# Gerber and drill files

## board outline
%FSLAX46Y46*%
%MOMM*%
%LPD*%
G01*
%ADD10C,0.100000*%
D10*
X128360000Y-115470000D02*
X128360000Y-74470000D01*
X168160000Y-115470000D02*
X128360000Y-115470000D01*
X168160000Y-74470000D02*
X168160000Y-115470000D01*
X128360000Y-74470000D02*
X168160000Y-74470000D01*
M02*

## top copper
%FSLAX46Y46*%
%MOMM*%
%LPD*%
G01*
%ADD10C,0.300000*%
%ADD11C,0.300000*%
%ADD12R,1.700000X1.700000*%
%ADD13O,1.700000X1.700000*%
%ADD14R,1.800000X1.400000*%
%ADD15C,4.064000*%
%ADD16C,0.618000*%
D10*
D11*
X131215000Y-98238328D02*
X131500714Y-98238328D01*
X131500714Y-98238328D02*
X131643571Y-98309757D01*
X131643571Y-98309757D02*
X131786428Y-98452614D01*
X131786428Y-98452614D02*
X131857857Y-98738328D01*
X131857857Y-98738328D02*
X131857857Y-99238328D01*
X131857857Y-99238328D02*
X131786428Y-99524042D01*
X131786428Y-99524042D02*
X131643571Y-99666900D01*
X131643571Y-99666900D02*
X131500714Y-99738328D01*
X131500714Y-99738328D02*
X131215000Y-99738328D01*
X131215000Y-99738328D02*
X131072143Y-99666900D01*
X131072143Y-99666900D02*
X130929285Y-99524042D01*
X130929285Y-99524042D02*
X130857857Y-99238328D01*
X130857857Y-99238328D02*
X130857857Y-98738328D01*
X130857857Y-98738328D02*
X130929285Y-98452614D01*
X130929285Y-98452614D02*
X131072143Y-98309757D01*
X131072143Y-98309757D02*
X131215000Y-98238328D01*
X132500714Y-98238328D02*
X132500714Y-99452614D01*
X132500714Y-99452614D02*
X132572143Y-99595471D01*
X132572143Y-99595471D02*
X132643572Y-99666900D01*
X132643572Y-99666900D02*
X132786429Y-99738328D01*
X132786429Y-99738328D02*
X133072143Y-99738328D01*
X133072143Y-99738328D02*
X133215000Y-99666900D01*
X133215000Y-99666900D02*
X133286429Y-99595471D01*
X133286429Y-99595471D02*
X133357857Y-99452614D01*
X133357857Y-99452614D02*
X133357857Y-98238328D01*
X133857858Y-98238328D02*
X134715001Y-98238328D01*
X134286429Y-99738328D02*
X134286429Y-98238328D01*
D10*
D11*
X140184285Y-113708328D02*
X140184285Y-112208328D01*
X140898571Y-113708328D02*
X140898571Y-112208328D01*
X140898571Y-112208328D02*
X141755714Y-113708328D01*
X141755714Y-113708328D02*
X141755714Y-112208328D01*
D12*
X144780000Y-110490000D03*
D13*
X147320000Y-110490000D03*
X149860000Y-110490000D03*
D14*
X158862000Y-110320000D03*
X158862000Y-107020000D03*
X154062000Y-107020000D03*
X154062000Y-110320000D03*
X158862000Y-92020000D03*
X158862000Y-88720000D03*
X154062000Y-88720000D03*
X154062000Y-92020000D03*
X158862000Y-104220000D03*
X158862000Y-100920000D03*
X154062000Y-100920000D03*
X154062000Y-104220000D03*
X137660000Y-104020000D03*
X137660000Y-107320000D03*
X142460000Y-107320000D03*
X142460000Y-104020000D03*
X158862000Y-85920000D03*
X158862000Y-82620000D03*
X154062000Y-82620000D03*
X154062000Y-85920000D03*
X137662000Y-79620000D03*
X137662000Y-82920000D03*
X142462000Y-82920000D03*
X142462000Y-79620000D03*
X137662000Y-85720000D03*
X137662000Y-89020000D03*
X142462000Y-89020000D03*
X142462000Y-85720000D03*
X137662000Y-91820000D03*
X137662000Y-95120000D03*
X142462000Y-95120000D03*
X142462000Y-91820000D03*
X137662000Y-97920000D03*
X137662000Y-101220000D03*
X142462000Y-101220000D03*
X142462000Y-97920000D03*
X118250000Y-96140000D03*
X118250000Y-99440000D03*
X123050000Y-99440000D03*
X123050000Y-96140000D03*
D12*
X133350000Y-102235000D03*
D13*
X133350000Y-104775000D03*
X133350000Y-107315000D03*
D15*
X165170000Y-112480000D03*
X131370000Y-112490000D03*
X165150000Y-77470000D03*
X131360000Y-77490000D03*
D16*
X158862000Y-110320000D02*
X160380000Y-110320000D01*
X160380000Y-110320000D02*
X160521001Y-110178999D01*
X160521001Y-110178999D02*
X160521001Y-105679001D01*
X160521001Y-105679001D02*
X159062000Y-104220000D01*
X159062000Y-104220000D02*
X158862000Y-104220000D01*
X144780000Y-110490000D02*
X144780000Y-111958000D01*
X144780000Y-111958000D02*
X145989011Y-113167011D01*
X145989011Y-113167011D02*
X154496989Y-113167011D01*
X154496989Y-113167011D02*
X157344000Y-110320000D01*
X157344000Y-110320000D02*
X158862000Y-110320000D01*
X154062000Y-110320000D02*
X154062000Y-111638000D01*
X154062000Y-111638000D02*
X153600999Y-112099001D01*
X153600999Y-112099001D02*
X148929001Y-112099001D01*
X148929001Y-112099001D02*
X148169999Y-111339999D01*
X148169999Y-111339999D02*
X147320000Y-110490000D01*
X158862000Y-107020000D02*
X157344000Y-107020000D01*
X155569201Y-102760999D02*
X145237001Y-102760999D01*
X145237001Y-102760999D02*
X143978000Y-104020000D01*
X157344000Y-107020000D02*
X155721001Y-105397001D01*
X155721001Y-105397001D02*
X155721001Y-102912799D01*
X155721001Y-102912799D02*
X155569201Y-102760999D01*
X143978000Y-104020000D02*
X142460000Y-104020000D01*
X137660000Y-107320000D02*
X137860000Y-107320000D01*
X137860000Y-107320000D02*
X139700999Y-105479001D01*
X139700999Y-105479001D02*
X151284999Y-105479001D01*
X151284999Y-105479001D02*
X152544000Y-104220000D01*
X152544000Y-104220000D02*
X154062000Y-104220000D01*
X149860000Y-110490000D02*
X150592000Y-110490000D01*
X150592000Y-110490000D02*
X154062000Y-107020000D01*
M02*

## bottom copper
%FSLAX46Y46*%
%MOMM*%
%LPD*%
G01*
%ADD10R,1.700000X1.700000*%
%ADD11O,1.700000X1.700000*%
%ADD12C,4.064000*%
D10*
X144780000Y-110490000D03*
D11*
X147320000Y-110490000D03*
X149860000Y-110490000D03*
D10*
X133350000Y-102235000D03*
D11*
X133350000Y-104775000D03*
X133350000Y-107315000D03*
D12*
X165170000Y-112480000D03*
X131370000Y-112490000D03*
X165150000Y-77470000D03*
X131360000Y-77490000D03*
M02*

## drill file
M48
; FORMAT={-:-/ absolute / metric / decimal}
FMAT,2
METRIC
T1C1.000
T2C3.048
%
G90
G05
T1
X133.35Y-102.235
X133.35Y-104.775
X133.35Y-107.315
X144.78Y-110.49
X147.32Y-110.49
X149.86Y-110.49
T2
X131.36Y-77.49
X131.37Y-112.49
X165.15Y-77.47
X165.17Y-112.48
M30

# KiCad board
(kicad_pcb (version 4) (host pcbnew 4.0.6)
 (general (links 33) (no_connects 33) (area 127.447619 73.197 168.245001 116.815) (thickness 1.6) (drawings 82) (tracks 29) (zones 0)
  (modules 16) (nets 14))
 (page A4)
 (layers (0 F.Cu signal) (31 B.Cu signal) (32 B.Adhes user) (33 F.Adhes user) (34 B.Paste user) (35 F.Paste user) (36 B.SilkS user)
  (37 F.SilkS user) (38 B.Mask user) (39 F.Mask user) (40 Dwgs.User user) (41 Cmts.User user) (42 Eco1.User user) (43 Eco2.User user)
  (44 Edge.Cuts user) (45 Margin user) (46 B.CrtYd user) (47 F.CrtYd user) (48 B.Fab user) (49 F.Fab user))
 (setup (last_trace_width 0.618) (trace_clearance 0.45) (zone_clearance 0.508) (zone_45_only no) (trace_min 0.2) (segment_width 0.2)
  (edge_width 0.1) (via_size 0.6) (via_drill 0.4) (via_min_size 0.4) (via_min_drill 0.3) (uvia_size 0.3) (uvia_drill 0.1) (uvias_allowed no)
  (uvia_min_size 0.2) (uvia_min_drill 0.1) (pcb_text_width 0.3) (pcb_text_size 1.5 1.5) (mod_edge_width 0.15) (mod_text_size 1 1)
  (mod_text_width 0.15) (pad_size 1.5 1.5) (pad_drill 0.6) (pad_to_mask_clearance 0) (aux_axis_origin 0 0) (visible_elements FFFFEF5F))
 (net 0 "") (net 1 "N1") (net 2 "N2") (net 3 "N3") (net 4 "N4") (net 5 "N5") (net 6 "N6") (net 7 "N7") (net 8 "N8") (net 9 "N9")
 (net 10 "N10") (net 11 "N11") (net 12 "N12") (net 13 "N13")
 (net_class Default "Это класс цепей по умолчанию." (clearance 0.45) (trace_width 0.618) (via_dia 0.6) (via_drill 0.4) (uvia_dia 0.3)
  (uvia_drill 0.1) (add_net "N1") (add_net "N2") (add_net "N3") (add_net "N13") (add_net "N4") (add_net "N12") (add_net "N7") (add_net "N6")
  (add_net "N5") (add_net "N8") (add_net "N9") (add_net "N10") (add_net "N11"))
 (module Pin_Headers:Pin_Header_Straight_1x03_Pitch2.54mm (layer F.Cu) (at 144.78 110.49 90)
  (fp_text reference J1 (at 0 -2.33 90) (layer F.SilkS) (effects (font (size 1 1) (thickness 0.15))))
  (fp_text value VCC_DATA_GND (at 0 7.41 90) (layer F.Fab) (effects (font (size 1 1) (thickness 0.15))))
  (pad 1 thru_hole rect (at 0 0 90) (size 1.7 1.7) (drill 1) (layers *.Cu *.Mask) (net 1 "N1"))
  (pad 2 thru_hole oval (at 0 2.54 90) (size 1.7 1.7) (drill 1) (layers *.Cu *.Mask) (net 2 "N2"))
  (pad 3 thru_hole oval (at 0 5.08 90) (size 1.7 1.7) (drill 1) (layers *.Cu *.Mask) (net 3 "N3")))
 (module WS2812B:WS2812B (layer F.Cu) (at 156.462 108.67 270)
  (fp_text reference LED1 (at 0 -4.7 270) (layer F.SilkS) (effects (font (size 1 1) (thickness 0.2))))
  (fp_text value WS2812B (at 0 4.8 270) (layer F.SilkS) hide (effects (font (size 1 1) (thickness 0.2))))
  (pad 1 smd rect (at 1.65 -2.4 270) (size 1.4 1.8) (layers F.Cu F.Paste F.Mask) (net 1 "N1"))
  (pad 2 smd rect (at -1.65 -2.4 270) (size 1.4 1.8) (layers F.Cu F.Paste F.Mask) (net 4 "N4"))
  (pad 3 smd rect (at -1.65 2.4 270) (size 1.4 1.8) (layers F.Cu F.Paste F.Mask) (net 3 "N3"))
  (pad 4 smd rect (at 1.65 2.4 270) (size 1.4 1.8) (layers F.Cu F.Paste F.Mask) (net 2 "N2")))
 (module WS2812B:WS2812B (layer F.Cu) (at 156.462 90.37 270)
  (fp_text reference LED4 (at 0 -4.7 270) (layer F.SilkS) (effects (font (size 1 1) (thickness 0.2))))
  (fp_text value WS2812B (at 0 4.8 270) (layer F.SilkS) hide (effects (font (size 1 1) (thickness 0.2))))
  (pad 1 smd rect (at 1.65 -2.4 270) (size 1.4 1.8) (layers F.Cu F.Paste F.Mask) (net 1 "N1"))
  (pad 2 smd rect (at -1.65 -2.4 270) (size 1.4 1.8) (layers F.Cu F.Paste F.Mask) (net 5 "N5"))
  (pad 3 smd rect (at -1.65 2.4 270) (size 1.4 1.8) (layers F.Cu F.Paste F.Mask) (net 3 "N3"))
  (pad 4 smd rect (at 1.65 2.4 270) (size 1.4 1.8) (layers F.Cu F.Paste F.Mask) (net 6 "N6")))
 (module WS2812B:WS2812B (layer F.Cu) (at 156.462 102.57 270)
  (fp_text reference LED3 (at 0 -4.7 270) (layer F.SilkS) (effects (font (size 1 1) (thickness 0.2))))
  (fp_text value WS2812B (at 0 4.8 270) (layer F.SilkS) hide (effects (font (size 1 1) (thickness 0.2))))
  (pad 1 smd rect (at 1.65 -2.4 270) (size 1.4 1.8) (layers F.Cu F.Paste F.Mask) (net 1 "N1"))
  (pad 2 smd rect (at -1.65 -2.4 270) (size 1.4 1.8) (layers F.Cu F.Paste F.Mask) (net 6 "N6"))
  (pad 3 smd rect (at -1.65 2.4 270) (size 1.4 1.8) (layers F.Cu F.Paste F.Mask) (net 3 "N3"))
  (pad 4 smd rect (at 1.65 2.4 270) (size 1.4 1.8) (layers F.Cu F.Paste F.Mask) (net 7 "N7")))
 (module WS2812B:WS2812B (layer F.Cu) (at 140.06 105.67 90)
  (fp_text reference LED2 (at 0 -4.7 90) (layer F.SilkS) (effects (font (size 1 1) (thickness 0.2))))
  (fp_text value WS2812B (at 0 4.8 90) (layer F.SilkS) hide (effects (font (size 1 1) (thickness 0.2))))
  (pad 1 smd rect (at 1.65 -2.4 90) (size 1.4 1.8) (layers F.Cu F.Paste F.Mask) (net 1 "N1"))
  (pad 2 smd rect (at -1.65 -2.4 90) (size 1.4 1.8) (layers F.Cu F.Paste F.Mask) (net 7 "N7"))
  (pad 3 smd rect (at -1.65 2.4 90) (size 1.4 1.8) (layers F.Cu F.Paste F.Mask) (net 3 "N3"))
  (pad 4 smd rect (at 1.65 2.4 90) (size 1.4 1.8) (layers F.Cu F.Paste F.Mask) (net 4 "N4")))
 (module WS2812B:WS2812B (layer F.Cu) (at 156.462 84.27 270)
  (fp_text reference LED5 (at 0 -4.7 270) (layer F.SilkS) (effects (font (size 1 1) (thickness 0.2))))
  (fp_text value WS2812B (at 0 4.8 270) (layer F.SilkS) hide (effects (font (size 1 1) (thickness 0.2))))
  (pad 1 smd rect (at 1.65 -2.4 270) (size 1.4 1.8) (layers F.Cu F.Paste F.Mask) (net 1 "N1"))
  (pad 2 smd rect (at -1.65 -2.4 270) (size 1.4 1.8) (layers F.Cu F.Paste F.Mask) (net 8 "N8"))
  (pad 3 smd rect (at -1.65 2.4 270) (size 1.4 1.8) (layers F.Cu F.Paste F.Mask) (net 3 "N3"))
  (pad 4 smd rect (at 1.65 2.4 270) (size 1.4 1.8) (layers F.Cu F.Paste F.Mask) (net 5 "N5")))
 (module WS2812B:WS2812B (layer F.Cu) (at 140.062 81.27 90)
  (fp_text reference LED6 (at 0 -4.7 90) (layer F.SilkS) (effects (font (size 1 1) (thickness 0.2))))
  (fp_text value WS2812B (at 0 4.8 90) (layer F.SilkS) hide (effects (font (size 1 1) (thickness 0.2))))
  (pad 1 smd rect (at 1.65 -2.4 90) (size 1.4 1.8) (layers F.Cu F.Paste F.Mask) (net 1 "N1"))
  (pad 2 smd rect (at -1.65 -2.4 90) (size 1.4 1.8) (layers F.Cu F.Paste F.Mask) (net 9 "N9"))
  (pad 3 smd rect (at -1.65 2.4 90) (size 1.4 1.8) (layers F.Cu F.Paste F.Mask) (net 3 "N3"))
  (pad 4 smd rect (at 1.65 2.4 90) (size 1.4 1.8) (layers F.Cu F.Paste F.Mask) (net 8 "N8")))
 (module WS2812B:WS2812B (layer F.Cu) (at 140.062 87.37 90)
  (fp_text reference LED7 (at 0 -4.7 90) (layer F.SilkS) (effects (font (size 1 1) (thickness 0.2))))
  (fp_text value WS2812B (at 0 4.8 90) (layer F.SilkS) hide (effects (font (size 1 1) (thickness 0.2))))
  (pad 1 smd rect (at 1.65 -2.4 90) (size 1.4 1.8) (layers F.Cu F.Paste F.Mask) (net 1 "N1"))
  (pad 2 smd rect (at -1.65 -2.4 90) (size 1.4 1.8) (layers F.Cu F.Paste F.Mask) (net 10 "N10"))
  (pad 3 smd rect (at -1.65 2.4 90) (size 1.4 1.8) (layers F.Cu F.Paste F.Mask) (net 3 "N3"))
  (pad 4 smd rect (at 1.65 2.4 90) (size 1.4 1.8) (layers F.Cu F.Paste F.Mask) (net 9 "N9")))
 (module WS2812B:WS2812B (layer F.Cu) (at 140.062 93.47 90)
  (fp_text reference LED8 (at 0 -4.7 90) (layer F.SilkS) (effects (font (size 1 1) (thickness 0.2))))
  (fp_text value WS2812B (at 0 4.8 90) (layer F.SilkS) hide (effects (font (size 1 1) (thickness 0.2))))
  (pad 1 smd rect (at 1.65 -2.4 90) (size 1.4 1.8) (layers F.Cu F.Paste F.Mask) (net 1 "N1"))
  (pad 2 smd rect (at -1.65 -2.4 90) (size 1.4 1.8) (layers F.Cu F.Paste F.Mask) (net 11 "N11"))
  (pad 3 smd rect (at -1.65 2.4 90) (size 1.4 1.8) (layers F.Cu F.Paste F.Mask) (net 3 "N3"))
  (pad 4 smd rect (at 1.65 2.4 90) (size 1.4 1.8) (layers F.Cu F.Paste F.Mask) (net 10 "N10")))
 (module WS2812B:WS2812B (layer F.Cu) (at 140.062 99.57 90)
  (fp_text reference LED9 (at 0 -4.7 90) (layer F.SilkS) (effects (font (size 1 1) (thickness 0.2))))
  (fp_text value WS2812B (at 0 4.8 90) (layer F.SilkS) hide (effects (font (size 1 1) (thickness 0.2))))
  (pad 1 smd rect (at 1.65 -2.4 90) (size 1.4 1.8) (layers F.Cu F.Paste F.Mask) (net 1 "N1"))
  (pad 2 smd rect (at -1.65 -2.4 90) (size 1.4 1.8) (layers F.Cu F.Paste F.Mask) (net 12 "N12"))
  (pad 3 smd rect (at -1.65 2.4 90) (size 1.4 1.8) (layers F.Cu F.Paste F.Mask) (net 3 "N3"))
  (pad 4 smd rect (at 1.65 2.4 90) (size 1.4 1.8) (layers F.Cu F.Paste F.Mask) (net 11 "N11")))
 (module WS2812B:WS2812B (layer F.Cu) (at 120.65 97.79 90)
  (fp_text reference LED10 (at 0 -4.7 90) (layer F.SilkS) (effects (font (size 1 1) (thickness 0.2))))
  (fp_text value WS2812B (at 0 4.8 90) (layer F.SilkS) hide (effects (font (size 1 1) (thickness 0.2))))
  (pad 1 smd rect (at 1.65 -2.4 90) (size 1.4 1.8) (layers F.Cu F.Paste F.Mask) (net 1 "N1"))
  (pad 2 smd rect (at -1.65 -2.4 90) (size 1.4 1.8) (layers F.Cu F.Paste F.Mask) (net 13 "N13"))
  (pad 3 smd rect (at -1.65 2.4 90) (size 1.4 1.8) (layers F.Cu F.Paste F.Mask) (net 3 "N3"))
  (pad 4 smd rect (at 1.65 2.4 90) (size 1.4 1.8) (layers F.Cu F.Paste F.Mask) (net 12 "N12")))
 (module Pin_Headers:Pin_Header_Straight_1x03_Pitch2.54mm (layer F.Cu) (at 133.35 102.235)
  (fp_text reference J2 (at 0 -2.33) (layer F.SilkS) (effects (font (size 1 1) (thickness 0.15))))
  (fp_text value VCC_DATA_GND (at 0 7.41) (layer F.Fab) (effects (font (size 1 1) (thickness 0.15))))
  (pad 1 thru_hole rect (at 0 0) (size 1.7 1.7) (drill 1) (layers *.Cu *.Mask) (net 1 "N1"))
  (pad 2 thru_hole oval (at 0 2.54) (size 1.7 1.7) (drill 1) (layers *.Cu *.Mask) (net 13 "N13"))
  (pad 3 thru_hole oval (at 0 5.08) (size 1.7 1.7) (drill 1) (layers *.Cu *.Mask) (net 3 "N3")))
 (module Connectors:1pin (layer F.Cu) (at 165.17 112.48)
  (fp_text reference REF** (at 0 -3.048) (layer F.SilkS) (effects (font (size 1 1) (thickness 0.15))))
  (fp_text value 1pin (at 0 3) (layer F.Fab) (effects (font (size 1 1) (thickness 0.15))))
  (pad 1 thru_hole circle (at 0 0) (size 4.064 4.064) (drill 3.048) (layers *.Cu *.Mask)))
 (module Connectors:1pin (layer F.Cu) (at 131.37 112.49)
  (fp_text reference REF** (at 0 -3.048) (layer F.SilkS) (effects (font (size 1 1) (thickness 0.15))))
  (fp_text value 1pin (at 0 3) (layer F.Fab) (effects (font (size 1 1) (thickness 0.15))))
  (pad 1 thru_hole circle (at 0 0) (size 4.064 4.064) (drill 3.048) (layers *.Cu *.Mask)))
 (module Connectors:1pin (layer F.Cu) (at 165.15 77.47)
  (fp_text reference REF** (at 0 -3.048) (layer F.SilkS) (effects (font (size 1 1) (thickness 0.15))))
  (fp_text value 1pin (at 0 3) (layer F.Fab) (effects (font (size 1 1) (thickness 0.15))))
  (pad 1 thru_hole circle (at 0 0) (size 4.064 4.064) (drill 3.048) (layers *.Cu *.Mask)))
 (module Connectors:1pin (layer F.Cu) (at 131.36 77.49)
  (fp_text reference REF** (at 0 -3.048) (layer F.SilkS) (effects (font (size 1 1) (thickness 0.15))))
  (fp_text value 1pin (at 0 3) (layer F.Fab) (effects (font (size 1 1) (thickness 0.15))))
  (pad 1 thru_hole circle (at 0 0) (size 4.064 4.064) (drill 3.048) (layers *.Cu *.Mask)))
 (gr_line (start 128.36 115.47) (end 128.36 74.47) (layer Edge.Cuts) (width 0.1))
 (gr_line (start 168.16 115.47) (end 128.36 115.47) (layer Edge.Cuts) (width 0.1))
 (gr_line (start 168.16 74.47) (end 168.16 115.47) (layer Edge.Cuts) (width 0.1))
 (gr_line (start 128.36 74.47) (end 168.16 74.47) (layer Edge.Cuts) (width 0.1))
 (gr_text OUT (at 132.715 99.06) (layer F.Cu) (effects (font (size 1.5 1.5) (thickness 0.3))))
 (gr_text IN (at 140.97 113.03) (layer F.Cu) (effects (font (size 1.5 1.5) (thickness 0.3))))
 (segment (start 158.862 110.32) (end 160.38 110.32) (width 0.618) (layer F.Cu) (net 1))
 (segment (start 160.38 110.32) (end 160.521001 110.178999) (width 0.618) (layer F.Cu) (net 1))
 (segment (start 160.521001 110.178999) (end 160.521001 105.679001) (width 0.618) (layer F.Cu) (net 1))
 (segment (start 160.521001 105.679001) (end 159.062 104.22) (width 0.618) (layer F.Cu) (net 1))
 (segment (start 159.062 104.22) (end 158.862 104.22) (width 0.618) (layer F.Cu) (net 1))
 (segment (start 144.78 110.49) (end 144.78 111.958) (width 0.618) (layer F.Cu) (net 1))
 (segment (start 144.78 111.958) (end 145.989011 113.167011) (width 0.618) (layer F.Cu) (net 1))
 (segment (start 145.989011 113.167011) (end 154.496989 113.167011) (width 0.618) (layer F.Cu) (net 1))
 (segment (start 154.496989 113.167011) (end 157.344 110.32) (width 0.618) (layer F.Cu) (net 1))
 (segment (start 157.344 110.32) (end 158.862 110.32) (width 0.618) (layer F.Cu) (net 1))
 (segment (start 154.062 110.32) (end 154.062 111.638) (width 0.618) (layer F.Cu) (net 2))
 (segment (start 154.062 111.638) (end 153.600999 112.099001) (width 0.618) (layer F.Cu) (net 2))
 (segment (start 153.600999 112.099001) (end 148.929001 112.099001) (width 0.618) (layer F.Cu) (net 2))
 (segment (start 148.929001 112.099001) (end 148.169999 111.339999) (width 0.618) (layer F.Cu) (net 2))
 (segment (start 148.169999 111.339999) (end 147.32 110.49) (width 0.618) (layer F.Cu) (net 2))
 (segment (start 158.862 107.02) (end 157.344 107.02) (width 0.618) (layer F.Cu) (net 4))
 (segment (start 155.569201 102.760999) (end 145.237001 102.760999) (width 0.618) (layer F.Cu) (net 4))
 (segment (start 145.237001 102.760999) (end 143.978 104.02) (width 0.618) (layer F.Cu) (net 4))
 (segment (start 157.344 107.02) (end 155.721001 105.397001) (width 0.618) (layer F.Cu) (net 4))
 (segment (start 155.721001 105.397001) (end 155.721001 102.912799) (width 0.618) (layer F.Cu) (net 4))
 (segment (start 155.721001 102.912799) (end 155.569201 102.760999) (width 0.618) (layer F.Cu) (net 4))
 (segment (start 143.978 104.02) (end 142.46 104.02) (width 0.618) (layer F.Cu) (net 4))
 (segment (start 137.66 107.32) (end 137.86 107.32) (width 0.618) (layer F.Cu) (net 7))
 (segment (start 137.86 107.32) (end 139.700999 105.479001) (width 0.618) (layer F.Cu) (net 7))
 (segment (start 139.700999 105.479001) (end 151.284999 105.479001) (width 0.618) (layer F.Cu) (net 7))
 (segment (start 151.284999 105.479001) (end 152.544 104.22) (width 0.618) (layer F.Cu) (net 7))
 (segment (start 152.544 104.22) (end 154.062 104.22) (width 0.618) (layer F.Cu) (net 7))
 (segment (start 149.86 110.49) (end 150.592 110.49) (width 0.618) (layer F.Cu) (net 3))
 (segment (start 150.592 110.49) (end 154.062 107.02) (width 0.618) (layer F.Cu) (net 3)))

